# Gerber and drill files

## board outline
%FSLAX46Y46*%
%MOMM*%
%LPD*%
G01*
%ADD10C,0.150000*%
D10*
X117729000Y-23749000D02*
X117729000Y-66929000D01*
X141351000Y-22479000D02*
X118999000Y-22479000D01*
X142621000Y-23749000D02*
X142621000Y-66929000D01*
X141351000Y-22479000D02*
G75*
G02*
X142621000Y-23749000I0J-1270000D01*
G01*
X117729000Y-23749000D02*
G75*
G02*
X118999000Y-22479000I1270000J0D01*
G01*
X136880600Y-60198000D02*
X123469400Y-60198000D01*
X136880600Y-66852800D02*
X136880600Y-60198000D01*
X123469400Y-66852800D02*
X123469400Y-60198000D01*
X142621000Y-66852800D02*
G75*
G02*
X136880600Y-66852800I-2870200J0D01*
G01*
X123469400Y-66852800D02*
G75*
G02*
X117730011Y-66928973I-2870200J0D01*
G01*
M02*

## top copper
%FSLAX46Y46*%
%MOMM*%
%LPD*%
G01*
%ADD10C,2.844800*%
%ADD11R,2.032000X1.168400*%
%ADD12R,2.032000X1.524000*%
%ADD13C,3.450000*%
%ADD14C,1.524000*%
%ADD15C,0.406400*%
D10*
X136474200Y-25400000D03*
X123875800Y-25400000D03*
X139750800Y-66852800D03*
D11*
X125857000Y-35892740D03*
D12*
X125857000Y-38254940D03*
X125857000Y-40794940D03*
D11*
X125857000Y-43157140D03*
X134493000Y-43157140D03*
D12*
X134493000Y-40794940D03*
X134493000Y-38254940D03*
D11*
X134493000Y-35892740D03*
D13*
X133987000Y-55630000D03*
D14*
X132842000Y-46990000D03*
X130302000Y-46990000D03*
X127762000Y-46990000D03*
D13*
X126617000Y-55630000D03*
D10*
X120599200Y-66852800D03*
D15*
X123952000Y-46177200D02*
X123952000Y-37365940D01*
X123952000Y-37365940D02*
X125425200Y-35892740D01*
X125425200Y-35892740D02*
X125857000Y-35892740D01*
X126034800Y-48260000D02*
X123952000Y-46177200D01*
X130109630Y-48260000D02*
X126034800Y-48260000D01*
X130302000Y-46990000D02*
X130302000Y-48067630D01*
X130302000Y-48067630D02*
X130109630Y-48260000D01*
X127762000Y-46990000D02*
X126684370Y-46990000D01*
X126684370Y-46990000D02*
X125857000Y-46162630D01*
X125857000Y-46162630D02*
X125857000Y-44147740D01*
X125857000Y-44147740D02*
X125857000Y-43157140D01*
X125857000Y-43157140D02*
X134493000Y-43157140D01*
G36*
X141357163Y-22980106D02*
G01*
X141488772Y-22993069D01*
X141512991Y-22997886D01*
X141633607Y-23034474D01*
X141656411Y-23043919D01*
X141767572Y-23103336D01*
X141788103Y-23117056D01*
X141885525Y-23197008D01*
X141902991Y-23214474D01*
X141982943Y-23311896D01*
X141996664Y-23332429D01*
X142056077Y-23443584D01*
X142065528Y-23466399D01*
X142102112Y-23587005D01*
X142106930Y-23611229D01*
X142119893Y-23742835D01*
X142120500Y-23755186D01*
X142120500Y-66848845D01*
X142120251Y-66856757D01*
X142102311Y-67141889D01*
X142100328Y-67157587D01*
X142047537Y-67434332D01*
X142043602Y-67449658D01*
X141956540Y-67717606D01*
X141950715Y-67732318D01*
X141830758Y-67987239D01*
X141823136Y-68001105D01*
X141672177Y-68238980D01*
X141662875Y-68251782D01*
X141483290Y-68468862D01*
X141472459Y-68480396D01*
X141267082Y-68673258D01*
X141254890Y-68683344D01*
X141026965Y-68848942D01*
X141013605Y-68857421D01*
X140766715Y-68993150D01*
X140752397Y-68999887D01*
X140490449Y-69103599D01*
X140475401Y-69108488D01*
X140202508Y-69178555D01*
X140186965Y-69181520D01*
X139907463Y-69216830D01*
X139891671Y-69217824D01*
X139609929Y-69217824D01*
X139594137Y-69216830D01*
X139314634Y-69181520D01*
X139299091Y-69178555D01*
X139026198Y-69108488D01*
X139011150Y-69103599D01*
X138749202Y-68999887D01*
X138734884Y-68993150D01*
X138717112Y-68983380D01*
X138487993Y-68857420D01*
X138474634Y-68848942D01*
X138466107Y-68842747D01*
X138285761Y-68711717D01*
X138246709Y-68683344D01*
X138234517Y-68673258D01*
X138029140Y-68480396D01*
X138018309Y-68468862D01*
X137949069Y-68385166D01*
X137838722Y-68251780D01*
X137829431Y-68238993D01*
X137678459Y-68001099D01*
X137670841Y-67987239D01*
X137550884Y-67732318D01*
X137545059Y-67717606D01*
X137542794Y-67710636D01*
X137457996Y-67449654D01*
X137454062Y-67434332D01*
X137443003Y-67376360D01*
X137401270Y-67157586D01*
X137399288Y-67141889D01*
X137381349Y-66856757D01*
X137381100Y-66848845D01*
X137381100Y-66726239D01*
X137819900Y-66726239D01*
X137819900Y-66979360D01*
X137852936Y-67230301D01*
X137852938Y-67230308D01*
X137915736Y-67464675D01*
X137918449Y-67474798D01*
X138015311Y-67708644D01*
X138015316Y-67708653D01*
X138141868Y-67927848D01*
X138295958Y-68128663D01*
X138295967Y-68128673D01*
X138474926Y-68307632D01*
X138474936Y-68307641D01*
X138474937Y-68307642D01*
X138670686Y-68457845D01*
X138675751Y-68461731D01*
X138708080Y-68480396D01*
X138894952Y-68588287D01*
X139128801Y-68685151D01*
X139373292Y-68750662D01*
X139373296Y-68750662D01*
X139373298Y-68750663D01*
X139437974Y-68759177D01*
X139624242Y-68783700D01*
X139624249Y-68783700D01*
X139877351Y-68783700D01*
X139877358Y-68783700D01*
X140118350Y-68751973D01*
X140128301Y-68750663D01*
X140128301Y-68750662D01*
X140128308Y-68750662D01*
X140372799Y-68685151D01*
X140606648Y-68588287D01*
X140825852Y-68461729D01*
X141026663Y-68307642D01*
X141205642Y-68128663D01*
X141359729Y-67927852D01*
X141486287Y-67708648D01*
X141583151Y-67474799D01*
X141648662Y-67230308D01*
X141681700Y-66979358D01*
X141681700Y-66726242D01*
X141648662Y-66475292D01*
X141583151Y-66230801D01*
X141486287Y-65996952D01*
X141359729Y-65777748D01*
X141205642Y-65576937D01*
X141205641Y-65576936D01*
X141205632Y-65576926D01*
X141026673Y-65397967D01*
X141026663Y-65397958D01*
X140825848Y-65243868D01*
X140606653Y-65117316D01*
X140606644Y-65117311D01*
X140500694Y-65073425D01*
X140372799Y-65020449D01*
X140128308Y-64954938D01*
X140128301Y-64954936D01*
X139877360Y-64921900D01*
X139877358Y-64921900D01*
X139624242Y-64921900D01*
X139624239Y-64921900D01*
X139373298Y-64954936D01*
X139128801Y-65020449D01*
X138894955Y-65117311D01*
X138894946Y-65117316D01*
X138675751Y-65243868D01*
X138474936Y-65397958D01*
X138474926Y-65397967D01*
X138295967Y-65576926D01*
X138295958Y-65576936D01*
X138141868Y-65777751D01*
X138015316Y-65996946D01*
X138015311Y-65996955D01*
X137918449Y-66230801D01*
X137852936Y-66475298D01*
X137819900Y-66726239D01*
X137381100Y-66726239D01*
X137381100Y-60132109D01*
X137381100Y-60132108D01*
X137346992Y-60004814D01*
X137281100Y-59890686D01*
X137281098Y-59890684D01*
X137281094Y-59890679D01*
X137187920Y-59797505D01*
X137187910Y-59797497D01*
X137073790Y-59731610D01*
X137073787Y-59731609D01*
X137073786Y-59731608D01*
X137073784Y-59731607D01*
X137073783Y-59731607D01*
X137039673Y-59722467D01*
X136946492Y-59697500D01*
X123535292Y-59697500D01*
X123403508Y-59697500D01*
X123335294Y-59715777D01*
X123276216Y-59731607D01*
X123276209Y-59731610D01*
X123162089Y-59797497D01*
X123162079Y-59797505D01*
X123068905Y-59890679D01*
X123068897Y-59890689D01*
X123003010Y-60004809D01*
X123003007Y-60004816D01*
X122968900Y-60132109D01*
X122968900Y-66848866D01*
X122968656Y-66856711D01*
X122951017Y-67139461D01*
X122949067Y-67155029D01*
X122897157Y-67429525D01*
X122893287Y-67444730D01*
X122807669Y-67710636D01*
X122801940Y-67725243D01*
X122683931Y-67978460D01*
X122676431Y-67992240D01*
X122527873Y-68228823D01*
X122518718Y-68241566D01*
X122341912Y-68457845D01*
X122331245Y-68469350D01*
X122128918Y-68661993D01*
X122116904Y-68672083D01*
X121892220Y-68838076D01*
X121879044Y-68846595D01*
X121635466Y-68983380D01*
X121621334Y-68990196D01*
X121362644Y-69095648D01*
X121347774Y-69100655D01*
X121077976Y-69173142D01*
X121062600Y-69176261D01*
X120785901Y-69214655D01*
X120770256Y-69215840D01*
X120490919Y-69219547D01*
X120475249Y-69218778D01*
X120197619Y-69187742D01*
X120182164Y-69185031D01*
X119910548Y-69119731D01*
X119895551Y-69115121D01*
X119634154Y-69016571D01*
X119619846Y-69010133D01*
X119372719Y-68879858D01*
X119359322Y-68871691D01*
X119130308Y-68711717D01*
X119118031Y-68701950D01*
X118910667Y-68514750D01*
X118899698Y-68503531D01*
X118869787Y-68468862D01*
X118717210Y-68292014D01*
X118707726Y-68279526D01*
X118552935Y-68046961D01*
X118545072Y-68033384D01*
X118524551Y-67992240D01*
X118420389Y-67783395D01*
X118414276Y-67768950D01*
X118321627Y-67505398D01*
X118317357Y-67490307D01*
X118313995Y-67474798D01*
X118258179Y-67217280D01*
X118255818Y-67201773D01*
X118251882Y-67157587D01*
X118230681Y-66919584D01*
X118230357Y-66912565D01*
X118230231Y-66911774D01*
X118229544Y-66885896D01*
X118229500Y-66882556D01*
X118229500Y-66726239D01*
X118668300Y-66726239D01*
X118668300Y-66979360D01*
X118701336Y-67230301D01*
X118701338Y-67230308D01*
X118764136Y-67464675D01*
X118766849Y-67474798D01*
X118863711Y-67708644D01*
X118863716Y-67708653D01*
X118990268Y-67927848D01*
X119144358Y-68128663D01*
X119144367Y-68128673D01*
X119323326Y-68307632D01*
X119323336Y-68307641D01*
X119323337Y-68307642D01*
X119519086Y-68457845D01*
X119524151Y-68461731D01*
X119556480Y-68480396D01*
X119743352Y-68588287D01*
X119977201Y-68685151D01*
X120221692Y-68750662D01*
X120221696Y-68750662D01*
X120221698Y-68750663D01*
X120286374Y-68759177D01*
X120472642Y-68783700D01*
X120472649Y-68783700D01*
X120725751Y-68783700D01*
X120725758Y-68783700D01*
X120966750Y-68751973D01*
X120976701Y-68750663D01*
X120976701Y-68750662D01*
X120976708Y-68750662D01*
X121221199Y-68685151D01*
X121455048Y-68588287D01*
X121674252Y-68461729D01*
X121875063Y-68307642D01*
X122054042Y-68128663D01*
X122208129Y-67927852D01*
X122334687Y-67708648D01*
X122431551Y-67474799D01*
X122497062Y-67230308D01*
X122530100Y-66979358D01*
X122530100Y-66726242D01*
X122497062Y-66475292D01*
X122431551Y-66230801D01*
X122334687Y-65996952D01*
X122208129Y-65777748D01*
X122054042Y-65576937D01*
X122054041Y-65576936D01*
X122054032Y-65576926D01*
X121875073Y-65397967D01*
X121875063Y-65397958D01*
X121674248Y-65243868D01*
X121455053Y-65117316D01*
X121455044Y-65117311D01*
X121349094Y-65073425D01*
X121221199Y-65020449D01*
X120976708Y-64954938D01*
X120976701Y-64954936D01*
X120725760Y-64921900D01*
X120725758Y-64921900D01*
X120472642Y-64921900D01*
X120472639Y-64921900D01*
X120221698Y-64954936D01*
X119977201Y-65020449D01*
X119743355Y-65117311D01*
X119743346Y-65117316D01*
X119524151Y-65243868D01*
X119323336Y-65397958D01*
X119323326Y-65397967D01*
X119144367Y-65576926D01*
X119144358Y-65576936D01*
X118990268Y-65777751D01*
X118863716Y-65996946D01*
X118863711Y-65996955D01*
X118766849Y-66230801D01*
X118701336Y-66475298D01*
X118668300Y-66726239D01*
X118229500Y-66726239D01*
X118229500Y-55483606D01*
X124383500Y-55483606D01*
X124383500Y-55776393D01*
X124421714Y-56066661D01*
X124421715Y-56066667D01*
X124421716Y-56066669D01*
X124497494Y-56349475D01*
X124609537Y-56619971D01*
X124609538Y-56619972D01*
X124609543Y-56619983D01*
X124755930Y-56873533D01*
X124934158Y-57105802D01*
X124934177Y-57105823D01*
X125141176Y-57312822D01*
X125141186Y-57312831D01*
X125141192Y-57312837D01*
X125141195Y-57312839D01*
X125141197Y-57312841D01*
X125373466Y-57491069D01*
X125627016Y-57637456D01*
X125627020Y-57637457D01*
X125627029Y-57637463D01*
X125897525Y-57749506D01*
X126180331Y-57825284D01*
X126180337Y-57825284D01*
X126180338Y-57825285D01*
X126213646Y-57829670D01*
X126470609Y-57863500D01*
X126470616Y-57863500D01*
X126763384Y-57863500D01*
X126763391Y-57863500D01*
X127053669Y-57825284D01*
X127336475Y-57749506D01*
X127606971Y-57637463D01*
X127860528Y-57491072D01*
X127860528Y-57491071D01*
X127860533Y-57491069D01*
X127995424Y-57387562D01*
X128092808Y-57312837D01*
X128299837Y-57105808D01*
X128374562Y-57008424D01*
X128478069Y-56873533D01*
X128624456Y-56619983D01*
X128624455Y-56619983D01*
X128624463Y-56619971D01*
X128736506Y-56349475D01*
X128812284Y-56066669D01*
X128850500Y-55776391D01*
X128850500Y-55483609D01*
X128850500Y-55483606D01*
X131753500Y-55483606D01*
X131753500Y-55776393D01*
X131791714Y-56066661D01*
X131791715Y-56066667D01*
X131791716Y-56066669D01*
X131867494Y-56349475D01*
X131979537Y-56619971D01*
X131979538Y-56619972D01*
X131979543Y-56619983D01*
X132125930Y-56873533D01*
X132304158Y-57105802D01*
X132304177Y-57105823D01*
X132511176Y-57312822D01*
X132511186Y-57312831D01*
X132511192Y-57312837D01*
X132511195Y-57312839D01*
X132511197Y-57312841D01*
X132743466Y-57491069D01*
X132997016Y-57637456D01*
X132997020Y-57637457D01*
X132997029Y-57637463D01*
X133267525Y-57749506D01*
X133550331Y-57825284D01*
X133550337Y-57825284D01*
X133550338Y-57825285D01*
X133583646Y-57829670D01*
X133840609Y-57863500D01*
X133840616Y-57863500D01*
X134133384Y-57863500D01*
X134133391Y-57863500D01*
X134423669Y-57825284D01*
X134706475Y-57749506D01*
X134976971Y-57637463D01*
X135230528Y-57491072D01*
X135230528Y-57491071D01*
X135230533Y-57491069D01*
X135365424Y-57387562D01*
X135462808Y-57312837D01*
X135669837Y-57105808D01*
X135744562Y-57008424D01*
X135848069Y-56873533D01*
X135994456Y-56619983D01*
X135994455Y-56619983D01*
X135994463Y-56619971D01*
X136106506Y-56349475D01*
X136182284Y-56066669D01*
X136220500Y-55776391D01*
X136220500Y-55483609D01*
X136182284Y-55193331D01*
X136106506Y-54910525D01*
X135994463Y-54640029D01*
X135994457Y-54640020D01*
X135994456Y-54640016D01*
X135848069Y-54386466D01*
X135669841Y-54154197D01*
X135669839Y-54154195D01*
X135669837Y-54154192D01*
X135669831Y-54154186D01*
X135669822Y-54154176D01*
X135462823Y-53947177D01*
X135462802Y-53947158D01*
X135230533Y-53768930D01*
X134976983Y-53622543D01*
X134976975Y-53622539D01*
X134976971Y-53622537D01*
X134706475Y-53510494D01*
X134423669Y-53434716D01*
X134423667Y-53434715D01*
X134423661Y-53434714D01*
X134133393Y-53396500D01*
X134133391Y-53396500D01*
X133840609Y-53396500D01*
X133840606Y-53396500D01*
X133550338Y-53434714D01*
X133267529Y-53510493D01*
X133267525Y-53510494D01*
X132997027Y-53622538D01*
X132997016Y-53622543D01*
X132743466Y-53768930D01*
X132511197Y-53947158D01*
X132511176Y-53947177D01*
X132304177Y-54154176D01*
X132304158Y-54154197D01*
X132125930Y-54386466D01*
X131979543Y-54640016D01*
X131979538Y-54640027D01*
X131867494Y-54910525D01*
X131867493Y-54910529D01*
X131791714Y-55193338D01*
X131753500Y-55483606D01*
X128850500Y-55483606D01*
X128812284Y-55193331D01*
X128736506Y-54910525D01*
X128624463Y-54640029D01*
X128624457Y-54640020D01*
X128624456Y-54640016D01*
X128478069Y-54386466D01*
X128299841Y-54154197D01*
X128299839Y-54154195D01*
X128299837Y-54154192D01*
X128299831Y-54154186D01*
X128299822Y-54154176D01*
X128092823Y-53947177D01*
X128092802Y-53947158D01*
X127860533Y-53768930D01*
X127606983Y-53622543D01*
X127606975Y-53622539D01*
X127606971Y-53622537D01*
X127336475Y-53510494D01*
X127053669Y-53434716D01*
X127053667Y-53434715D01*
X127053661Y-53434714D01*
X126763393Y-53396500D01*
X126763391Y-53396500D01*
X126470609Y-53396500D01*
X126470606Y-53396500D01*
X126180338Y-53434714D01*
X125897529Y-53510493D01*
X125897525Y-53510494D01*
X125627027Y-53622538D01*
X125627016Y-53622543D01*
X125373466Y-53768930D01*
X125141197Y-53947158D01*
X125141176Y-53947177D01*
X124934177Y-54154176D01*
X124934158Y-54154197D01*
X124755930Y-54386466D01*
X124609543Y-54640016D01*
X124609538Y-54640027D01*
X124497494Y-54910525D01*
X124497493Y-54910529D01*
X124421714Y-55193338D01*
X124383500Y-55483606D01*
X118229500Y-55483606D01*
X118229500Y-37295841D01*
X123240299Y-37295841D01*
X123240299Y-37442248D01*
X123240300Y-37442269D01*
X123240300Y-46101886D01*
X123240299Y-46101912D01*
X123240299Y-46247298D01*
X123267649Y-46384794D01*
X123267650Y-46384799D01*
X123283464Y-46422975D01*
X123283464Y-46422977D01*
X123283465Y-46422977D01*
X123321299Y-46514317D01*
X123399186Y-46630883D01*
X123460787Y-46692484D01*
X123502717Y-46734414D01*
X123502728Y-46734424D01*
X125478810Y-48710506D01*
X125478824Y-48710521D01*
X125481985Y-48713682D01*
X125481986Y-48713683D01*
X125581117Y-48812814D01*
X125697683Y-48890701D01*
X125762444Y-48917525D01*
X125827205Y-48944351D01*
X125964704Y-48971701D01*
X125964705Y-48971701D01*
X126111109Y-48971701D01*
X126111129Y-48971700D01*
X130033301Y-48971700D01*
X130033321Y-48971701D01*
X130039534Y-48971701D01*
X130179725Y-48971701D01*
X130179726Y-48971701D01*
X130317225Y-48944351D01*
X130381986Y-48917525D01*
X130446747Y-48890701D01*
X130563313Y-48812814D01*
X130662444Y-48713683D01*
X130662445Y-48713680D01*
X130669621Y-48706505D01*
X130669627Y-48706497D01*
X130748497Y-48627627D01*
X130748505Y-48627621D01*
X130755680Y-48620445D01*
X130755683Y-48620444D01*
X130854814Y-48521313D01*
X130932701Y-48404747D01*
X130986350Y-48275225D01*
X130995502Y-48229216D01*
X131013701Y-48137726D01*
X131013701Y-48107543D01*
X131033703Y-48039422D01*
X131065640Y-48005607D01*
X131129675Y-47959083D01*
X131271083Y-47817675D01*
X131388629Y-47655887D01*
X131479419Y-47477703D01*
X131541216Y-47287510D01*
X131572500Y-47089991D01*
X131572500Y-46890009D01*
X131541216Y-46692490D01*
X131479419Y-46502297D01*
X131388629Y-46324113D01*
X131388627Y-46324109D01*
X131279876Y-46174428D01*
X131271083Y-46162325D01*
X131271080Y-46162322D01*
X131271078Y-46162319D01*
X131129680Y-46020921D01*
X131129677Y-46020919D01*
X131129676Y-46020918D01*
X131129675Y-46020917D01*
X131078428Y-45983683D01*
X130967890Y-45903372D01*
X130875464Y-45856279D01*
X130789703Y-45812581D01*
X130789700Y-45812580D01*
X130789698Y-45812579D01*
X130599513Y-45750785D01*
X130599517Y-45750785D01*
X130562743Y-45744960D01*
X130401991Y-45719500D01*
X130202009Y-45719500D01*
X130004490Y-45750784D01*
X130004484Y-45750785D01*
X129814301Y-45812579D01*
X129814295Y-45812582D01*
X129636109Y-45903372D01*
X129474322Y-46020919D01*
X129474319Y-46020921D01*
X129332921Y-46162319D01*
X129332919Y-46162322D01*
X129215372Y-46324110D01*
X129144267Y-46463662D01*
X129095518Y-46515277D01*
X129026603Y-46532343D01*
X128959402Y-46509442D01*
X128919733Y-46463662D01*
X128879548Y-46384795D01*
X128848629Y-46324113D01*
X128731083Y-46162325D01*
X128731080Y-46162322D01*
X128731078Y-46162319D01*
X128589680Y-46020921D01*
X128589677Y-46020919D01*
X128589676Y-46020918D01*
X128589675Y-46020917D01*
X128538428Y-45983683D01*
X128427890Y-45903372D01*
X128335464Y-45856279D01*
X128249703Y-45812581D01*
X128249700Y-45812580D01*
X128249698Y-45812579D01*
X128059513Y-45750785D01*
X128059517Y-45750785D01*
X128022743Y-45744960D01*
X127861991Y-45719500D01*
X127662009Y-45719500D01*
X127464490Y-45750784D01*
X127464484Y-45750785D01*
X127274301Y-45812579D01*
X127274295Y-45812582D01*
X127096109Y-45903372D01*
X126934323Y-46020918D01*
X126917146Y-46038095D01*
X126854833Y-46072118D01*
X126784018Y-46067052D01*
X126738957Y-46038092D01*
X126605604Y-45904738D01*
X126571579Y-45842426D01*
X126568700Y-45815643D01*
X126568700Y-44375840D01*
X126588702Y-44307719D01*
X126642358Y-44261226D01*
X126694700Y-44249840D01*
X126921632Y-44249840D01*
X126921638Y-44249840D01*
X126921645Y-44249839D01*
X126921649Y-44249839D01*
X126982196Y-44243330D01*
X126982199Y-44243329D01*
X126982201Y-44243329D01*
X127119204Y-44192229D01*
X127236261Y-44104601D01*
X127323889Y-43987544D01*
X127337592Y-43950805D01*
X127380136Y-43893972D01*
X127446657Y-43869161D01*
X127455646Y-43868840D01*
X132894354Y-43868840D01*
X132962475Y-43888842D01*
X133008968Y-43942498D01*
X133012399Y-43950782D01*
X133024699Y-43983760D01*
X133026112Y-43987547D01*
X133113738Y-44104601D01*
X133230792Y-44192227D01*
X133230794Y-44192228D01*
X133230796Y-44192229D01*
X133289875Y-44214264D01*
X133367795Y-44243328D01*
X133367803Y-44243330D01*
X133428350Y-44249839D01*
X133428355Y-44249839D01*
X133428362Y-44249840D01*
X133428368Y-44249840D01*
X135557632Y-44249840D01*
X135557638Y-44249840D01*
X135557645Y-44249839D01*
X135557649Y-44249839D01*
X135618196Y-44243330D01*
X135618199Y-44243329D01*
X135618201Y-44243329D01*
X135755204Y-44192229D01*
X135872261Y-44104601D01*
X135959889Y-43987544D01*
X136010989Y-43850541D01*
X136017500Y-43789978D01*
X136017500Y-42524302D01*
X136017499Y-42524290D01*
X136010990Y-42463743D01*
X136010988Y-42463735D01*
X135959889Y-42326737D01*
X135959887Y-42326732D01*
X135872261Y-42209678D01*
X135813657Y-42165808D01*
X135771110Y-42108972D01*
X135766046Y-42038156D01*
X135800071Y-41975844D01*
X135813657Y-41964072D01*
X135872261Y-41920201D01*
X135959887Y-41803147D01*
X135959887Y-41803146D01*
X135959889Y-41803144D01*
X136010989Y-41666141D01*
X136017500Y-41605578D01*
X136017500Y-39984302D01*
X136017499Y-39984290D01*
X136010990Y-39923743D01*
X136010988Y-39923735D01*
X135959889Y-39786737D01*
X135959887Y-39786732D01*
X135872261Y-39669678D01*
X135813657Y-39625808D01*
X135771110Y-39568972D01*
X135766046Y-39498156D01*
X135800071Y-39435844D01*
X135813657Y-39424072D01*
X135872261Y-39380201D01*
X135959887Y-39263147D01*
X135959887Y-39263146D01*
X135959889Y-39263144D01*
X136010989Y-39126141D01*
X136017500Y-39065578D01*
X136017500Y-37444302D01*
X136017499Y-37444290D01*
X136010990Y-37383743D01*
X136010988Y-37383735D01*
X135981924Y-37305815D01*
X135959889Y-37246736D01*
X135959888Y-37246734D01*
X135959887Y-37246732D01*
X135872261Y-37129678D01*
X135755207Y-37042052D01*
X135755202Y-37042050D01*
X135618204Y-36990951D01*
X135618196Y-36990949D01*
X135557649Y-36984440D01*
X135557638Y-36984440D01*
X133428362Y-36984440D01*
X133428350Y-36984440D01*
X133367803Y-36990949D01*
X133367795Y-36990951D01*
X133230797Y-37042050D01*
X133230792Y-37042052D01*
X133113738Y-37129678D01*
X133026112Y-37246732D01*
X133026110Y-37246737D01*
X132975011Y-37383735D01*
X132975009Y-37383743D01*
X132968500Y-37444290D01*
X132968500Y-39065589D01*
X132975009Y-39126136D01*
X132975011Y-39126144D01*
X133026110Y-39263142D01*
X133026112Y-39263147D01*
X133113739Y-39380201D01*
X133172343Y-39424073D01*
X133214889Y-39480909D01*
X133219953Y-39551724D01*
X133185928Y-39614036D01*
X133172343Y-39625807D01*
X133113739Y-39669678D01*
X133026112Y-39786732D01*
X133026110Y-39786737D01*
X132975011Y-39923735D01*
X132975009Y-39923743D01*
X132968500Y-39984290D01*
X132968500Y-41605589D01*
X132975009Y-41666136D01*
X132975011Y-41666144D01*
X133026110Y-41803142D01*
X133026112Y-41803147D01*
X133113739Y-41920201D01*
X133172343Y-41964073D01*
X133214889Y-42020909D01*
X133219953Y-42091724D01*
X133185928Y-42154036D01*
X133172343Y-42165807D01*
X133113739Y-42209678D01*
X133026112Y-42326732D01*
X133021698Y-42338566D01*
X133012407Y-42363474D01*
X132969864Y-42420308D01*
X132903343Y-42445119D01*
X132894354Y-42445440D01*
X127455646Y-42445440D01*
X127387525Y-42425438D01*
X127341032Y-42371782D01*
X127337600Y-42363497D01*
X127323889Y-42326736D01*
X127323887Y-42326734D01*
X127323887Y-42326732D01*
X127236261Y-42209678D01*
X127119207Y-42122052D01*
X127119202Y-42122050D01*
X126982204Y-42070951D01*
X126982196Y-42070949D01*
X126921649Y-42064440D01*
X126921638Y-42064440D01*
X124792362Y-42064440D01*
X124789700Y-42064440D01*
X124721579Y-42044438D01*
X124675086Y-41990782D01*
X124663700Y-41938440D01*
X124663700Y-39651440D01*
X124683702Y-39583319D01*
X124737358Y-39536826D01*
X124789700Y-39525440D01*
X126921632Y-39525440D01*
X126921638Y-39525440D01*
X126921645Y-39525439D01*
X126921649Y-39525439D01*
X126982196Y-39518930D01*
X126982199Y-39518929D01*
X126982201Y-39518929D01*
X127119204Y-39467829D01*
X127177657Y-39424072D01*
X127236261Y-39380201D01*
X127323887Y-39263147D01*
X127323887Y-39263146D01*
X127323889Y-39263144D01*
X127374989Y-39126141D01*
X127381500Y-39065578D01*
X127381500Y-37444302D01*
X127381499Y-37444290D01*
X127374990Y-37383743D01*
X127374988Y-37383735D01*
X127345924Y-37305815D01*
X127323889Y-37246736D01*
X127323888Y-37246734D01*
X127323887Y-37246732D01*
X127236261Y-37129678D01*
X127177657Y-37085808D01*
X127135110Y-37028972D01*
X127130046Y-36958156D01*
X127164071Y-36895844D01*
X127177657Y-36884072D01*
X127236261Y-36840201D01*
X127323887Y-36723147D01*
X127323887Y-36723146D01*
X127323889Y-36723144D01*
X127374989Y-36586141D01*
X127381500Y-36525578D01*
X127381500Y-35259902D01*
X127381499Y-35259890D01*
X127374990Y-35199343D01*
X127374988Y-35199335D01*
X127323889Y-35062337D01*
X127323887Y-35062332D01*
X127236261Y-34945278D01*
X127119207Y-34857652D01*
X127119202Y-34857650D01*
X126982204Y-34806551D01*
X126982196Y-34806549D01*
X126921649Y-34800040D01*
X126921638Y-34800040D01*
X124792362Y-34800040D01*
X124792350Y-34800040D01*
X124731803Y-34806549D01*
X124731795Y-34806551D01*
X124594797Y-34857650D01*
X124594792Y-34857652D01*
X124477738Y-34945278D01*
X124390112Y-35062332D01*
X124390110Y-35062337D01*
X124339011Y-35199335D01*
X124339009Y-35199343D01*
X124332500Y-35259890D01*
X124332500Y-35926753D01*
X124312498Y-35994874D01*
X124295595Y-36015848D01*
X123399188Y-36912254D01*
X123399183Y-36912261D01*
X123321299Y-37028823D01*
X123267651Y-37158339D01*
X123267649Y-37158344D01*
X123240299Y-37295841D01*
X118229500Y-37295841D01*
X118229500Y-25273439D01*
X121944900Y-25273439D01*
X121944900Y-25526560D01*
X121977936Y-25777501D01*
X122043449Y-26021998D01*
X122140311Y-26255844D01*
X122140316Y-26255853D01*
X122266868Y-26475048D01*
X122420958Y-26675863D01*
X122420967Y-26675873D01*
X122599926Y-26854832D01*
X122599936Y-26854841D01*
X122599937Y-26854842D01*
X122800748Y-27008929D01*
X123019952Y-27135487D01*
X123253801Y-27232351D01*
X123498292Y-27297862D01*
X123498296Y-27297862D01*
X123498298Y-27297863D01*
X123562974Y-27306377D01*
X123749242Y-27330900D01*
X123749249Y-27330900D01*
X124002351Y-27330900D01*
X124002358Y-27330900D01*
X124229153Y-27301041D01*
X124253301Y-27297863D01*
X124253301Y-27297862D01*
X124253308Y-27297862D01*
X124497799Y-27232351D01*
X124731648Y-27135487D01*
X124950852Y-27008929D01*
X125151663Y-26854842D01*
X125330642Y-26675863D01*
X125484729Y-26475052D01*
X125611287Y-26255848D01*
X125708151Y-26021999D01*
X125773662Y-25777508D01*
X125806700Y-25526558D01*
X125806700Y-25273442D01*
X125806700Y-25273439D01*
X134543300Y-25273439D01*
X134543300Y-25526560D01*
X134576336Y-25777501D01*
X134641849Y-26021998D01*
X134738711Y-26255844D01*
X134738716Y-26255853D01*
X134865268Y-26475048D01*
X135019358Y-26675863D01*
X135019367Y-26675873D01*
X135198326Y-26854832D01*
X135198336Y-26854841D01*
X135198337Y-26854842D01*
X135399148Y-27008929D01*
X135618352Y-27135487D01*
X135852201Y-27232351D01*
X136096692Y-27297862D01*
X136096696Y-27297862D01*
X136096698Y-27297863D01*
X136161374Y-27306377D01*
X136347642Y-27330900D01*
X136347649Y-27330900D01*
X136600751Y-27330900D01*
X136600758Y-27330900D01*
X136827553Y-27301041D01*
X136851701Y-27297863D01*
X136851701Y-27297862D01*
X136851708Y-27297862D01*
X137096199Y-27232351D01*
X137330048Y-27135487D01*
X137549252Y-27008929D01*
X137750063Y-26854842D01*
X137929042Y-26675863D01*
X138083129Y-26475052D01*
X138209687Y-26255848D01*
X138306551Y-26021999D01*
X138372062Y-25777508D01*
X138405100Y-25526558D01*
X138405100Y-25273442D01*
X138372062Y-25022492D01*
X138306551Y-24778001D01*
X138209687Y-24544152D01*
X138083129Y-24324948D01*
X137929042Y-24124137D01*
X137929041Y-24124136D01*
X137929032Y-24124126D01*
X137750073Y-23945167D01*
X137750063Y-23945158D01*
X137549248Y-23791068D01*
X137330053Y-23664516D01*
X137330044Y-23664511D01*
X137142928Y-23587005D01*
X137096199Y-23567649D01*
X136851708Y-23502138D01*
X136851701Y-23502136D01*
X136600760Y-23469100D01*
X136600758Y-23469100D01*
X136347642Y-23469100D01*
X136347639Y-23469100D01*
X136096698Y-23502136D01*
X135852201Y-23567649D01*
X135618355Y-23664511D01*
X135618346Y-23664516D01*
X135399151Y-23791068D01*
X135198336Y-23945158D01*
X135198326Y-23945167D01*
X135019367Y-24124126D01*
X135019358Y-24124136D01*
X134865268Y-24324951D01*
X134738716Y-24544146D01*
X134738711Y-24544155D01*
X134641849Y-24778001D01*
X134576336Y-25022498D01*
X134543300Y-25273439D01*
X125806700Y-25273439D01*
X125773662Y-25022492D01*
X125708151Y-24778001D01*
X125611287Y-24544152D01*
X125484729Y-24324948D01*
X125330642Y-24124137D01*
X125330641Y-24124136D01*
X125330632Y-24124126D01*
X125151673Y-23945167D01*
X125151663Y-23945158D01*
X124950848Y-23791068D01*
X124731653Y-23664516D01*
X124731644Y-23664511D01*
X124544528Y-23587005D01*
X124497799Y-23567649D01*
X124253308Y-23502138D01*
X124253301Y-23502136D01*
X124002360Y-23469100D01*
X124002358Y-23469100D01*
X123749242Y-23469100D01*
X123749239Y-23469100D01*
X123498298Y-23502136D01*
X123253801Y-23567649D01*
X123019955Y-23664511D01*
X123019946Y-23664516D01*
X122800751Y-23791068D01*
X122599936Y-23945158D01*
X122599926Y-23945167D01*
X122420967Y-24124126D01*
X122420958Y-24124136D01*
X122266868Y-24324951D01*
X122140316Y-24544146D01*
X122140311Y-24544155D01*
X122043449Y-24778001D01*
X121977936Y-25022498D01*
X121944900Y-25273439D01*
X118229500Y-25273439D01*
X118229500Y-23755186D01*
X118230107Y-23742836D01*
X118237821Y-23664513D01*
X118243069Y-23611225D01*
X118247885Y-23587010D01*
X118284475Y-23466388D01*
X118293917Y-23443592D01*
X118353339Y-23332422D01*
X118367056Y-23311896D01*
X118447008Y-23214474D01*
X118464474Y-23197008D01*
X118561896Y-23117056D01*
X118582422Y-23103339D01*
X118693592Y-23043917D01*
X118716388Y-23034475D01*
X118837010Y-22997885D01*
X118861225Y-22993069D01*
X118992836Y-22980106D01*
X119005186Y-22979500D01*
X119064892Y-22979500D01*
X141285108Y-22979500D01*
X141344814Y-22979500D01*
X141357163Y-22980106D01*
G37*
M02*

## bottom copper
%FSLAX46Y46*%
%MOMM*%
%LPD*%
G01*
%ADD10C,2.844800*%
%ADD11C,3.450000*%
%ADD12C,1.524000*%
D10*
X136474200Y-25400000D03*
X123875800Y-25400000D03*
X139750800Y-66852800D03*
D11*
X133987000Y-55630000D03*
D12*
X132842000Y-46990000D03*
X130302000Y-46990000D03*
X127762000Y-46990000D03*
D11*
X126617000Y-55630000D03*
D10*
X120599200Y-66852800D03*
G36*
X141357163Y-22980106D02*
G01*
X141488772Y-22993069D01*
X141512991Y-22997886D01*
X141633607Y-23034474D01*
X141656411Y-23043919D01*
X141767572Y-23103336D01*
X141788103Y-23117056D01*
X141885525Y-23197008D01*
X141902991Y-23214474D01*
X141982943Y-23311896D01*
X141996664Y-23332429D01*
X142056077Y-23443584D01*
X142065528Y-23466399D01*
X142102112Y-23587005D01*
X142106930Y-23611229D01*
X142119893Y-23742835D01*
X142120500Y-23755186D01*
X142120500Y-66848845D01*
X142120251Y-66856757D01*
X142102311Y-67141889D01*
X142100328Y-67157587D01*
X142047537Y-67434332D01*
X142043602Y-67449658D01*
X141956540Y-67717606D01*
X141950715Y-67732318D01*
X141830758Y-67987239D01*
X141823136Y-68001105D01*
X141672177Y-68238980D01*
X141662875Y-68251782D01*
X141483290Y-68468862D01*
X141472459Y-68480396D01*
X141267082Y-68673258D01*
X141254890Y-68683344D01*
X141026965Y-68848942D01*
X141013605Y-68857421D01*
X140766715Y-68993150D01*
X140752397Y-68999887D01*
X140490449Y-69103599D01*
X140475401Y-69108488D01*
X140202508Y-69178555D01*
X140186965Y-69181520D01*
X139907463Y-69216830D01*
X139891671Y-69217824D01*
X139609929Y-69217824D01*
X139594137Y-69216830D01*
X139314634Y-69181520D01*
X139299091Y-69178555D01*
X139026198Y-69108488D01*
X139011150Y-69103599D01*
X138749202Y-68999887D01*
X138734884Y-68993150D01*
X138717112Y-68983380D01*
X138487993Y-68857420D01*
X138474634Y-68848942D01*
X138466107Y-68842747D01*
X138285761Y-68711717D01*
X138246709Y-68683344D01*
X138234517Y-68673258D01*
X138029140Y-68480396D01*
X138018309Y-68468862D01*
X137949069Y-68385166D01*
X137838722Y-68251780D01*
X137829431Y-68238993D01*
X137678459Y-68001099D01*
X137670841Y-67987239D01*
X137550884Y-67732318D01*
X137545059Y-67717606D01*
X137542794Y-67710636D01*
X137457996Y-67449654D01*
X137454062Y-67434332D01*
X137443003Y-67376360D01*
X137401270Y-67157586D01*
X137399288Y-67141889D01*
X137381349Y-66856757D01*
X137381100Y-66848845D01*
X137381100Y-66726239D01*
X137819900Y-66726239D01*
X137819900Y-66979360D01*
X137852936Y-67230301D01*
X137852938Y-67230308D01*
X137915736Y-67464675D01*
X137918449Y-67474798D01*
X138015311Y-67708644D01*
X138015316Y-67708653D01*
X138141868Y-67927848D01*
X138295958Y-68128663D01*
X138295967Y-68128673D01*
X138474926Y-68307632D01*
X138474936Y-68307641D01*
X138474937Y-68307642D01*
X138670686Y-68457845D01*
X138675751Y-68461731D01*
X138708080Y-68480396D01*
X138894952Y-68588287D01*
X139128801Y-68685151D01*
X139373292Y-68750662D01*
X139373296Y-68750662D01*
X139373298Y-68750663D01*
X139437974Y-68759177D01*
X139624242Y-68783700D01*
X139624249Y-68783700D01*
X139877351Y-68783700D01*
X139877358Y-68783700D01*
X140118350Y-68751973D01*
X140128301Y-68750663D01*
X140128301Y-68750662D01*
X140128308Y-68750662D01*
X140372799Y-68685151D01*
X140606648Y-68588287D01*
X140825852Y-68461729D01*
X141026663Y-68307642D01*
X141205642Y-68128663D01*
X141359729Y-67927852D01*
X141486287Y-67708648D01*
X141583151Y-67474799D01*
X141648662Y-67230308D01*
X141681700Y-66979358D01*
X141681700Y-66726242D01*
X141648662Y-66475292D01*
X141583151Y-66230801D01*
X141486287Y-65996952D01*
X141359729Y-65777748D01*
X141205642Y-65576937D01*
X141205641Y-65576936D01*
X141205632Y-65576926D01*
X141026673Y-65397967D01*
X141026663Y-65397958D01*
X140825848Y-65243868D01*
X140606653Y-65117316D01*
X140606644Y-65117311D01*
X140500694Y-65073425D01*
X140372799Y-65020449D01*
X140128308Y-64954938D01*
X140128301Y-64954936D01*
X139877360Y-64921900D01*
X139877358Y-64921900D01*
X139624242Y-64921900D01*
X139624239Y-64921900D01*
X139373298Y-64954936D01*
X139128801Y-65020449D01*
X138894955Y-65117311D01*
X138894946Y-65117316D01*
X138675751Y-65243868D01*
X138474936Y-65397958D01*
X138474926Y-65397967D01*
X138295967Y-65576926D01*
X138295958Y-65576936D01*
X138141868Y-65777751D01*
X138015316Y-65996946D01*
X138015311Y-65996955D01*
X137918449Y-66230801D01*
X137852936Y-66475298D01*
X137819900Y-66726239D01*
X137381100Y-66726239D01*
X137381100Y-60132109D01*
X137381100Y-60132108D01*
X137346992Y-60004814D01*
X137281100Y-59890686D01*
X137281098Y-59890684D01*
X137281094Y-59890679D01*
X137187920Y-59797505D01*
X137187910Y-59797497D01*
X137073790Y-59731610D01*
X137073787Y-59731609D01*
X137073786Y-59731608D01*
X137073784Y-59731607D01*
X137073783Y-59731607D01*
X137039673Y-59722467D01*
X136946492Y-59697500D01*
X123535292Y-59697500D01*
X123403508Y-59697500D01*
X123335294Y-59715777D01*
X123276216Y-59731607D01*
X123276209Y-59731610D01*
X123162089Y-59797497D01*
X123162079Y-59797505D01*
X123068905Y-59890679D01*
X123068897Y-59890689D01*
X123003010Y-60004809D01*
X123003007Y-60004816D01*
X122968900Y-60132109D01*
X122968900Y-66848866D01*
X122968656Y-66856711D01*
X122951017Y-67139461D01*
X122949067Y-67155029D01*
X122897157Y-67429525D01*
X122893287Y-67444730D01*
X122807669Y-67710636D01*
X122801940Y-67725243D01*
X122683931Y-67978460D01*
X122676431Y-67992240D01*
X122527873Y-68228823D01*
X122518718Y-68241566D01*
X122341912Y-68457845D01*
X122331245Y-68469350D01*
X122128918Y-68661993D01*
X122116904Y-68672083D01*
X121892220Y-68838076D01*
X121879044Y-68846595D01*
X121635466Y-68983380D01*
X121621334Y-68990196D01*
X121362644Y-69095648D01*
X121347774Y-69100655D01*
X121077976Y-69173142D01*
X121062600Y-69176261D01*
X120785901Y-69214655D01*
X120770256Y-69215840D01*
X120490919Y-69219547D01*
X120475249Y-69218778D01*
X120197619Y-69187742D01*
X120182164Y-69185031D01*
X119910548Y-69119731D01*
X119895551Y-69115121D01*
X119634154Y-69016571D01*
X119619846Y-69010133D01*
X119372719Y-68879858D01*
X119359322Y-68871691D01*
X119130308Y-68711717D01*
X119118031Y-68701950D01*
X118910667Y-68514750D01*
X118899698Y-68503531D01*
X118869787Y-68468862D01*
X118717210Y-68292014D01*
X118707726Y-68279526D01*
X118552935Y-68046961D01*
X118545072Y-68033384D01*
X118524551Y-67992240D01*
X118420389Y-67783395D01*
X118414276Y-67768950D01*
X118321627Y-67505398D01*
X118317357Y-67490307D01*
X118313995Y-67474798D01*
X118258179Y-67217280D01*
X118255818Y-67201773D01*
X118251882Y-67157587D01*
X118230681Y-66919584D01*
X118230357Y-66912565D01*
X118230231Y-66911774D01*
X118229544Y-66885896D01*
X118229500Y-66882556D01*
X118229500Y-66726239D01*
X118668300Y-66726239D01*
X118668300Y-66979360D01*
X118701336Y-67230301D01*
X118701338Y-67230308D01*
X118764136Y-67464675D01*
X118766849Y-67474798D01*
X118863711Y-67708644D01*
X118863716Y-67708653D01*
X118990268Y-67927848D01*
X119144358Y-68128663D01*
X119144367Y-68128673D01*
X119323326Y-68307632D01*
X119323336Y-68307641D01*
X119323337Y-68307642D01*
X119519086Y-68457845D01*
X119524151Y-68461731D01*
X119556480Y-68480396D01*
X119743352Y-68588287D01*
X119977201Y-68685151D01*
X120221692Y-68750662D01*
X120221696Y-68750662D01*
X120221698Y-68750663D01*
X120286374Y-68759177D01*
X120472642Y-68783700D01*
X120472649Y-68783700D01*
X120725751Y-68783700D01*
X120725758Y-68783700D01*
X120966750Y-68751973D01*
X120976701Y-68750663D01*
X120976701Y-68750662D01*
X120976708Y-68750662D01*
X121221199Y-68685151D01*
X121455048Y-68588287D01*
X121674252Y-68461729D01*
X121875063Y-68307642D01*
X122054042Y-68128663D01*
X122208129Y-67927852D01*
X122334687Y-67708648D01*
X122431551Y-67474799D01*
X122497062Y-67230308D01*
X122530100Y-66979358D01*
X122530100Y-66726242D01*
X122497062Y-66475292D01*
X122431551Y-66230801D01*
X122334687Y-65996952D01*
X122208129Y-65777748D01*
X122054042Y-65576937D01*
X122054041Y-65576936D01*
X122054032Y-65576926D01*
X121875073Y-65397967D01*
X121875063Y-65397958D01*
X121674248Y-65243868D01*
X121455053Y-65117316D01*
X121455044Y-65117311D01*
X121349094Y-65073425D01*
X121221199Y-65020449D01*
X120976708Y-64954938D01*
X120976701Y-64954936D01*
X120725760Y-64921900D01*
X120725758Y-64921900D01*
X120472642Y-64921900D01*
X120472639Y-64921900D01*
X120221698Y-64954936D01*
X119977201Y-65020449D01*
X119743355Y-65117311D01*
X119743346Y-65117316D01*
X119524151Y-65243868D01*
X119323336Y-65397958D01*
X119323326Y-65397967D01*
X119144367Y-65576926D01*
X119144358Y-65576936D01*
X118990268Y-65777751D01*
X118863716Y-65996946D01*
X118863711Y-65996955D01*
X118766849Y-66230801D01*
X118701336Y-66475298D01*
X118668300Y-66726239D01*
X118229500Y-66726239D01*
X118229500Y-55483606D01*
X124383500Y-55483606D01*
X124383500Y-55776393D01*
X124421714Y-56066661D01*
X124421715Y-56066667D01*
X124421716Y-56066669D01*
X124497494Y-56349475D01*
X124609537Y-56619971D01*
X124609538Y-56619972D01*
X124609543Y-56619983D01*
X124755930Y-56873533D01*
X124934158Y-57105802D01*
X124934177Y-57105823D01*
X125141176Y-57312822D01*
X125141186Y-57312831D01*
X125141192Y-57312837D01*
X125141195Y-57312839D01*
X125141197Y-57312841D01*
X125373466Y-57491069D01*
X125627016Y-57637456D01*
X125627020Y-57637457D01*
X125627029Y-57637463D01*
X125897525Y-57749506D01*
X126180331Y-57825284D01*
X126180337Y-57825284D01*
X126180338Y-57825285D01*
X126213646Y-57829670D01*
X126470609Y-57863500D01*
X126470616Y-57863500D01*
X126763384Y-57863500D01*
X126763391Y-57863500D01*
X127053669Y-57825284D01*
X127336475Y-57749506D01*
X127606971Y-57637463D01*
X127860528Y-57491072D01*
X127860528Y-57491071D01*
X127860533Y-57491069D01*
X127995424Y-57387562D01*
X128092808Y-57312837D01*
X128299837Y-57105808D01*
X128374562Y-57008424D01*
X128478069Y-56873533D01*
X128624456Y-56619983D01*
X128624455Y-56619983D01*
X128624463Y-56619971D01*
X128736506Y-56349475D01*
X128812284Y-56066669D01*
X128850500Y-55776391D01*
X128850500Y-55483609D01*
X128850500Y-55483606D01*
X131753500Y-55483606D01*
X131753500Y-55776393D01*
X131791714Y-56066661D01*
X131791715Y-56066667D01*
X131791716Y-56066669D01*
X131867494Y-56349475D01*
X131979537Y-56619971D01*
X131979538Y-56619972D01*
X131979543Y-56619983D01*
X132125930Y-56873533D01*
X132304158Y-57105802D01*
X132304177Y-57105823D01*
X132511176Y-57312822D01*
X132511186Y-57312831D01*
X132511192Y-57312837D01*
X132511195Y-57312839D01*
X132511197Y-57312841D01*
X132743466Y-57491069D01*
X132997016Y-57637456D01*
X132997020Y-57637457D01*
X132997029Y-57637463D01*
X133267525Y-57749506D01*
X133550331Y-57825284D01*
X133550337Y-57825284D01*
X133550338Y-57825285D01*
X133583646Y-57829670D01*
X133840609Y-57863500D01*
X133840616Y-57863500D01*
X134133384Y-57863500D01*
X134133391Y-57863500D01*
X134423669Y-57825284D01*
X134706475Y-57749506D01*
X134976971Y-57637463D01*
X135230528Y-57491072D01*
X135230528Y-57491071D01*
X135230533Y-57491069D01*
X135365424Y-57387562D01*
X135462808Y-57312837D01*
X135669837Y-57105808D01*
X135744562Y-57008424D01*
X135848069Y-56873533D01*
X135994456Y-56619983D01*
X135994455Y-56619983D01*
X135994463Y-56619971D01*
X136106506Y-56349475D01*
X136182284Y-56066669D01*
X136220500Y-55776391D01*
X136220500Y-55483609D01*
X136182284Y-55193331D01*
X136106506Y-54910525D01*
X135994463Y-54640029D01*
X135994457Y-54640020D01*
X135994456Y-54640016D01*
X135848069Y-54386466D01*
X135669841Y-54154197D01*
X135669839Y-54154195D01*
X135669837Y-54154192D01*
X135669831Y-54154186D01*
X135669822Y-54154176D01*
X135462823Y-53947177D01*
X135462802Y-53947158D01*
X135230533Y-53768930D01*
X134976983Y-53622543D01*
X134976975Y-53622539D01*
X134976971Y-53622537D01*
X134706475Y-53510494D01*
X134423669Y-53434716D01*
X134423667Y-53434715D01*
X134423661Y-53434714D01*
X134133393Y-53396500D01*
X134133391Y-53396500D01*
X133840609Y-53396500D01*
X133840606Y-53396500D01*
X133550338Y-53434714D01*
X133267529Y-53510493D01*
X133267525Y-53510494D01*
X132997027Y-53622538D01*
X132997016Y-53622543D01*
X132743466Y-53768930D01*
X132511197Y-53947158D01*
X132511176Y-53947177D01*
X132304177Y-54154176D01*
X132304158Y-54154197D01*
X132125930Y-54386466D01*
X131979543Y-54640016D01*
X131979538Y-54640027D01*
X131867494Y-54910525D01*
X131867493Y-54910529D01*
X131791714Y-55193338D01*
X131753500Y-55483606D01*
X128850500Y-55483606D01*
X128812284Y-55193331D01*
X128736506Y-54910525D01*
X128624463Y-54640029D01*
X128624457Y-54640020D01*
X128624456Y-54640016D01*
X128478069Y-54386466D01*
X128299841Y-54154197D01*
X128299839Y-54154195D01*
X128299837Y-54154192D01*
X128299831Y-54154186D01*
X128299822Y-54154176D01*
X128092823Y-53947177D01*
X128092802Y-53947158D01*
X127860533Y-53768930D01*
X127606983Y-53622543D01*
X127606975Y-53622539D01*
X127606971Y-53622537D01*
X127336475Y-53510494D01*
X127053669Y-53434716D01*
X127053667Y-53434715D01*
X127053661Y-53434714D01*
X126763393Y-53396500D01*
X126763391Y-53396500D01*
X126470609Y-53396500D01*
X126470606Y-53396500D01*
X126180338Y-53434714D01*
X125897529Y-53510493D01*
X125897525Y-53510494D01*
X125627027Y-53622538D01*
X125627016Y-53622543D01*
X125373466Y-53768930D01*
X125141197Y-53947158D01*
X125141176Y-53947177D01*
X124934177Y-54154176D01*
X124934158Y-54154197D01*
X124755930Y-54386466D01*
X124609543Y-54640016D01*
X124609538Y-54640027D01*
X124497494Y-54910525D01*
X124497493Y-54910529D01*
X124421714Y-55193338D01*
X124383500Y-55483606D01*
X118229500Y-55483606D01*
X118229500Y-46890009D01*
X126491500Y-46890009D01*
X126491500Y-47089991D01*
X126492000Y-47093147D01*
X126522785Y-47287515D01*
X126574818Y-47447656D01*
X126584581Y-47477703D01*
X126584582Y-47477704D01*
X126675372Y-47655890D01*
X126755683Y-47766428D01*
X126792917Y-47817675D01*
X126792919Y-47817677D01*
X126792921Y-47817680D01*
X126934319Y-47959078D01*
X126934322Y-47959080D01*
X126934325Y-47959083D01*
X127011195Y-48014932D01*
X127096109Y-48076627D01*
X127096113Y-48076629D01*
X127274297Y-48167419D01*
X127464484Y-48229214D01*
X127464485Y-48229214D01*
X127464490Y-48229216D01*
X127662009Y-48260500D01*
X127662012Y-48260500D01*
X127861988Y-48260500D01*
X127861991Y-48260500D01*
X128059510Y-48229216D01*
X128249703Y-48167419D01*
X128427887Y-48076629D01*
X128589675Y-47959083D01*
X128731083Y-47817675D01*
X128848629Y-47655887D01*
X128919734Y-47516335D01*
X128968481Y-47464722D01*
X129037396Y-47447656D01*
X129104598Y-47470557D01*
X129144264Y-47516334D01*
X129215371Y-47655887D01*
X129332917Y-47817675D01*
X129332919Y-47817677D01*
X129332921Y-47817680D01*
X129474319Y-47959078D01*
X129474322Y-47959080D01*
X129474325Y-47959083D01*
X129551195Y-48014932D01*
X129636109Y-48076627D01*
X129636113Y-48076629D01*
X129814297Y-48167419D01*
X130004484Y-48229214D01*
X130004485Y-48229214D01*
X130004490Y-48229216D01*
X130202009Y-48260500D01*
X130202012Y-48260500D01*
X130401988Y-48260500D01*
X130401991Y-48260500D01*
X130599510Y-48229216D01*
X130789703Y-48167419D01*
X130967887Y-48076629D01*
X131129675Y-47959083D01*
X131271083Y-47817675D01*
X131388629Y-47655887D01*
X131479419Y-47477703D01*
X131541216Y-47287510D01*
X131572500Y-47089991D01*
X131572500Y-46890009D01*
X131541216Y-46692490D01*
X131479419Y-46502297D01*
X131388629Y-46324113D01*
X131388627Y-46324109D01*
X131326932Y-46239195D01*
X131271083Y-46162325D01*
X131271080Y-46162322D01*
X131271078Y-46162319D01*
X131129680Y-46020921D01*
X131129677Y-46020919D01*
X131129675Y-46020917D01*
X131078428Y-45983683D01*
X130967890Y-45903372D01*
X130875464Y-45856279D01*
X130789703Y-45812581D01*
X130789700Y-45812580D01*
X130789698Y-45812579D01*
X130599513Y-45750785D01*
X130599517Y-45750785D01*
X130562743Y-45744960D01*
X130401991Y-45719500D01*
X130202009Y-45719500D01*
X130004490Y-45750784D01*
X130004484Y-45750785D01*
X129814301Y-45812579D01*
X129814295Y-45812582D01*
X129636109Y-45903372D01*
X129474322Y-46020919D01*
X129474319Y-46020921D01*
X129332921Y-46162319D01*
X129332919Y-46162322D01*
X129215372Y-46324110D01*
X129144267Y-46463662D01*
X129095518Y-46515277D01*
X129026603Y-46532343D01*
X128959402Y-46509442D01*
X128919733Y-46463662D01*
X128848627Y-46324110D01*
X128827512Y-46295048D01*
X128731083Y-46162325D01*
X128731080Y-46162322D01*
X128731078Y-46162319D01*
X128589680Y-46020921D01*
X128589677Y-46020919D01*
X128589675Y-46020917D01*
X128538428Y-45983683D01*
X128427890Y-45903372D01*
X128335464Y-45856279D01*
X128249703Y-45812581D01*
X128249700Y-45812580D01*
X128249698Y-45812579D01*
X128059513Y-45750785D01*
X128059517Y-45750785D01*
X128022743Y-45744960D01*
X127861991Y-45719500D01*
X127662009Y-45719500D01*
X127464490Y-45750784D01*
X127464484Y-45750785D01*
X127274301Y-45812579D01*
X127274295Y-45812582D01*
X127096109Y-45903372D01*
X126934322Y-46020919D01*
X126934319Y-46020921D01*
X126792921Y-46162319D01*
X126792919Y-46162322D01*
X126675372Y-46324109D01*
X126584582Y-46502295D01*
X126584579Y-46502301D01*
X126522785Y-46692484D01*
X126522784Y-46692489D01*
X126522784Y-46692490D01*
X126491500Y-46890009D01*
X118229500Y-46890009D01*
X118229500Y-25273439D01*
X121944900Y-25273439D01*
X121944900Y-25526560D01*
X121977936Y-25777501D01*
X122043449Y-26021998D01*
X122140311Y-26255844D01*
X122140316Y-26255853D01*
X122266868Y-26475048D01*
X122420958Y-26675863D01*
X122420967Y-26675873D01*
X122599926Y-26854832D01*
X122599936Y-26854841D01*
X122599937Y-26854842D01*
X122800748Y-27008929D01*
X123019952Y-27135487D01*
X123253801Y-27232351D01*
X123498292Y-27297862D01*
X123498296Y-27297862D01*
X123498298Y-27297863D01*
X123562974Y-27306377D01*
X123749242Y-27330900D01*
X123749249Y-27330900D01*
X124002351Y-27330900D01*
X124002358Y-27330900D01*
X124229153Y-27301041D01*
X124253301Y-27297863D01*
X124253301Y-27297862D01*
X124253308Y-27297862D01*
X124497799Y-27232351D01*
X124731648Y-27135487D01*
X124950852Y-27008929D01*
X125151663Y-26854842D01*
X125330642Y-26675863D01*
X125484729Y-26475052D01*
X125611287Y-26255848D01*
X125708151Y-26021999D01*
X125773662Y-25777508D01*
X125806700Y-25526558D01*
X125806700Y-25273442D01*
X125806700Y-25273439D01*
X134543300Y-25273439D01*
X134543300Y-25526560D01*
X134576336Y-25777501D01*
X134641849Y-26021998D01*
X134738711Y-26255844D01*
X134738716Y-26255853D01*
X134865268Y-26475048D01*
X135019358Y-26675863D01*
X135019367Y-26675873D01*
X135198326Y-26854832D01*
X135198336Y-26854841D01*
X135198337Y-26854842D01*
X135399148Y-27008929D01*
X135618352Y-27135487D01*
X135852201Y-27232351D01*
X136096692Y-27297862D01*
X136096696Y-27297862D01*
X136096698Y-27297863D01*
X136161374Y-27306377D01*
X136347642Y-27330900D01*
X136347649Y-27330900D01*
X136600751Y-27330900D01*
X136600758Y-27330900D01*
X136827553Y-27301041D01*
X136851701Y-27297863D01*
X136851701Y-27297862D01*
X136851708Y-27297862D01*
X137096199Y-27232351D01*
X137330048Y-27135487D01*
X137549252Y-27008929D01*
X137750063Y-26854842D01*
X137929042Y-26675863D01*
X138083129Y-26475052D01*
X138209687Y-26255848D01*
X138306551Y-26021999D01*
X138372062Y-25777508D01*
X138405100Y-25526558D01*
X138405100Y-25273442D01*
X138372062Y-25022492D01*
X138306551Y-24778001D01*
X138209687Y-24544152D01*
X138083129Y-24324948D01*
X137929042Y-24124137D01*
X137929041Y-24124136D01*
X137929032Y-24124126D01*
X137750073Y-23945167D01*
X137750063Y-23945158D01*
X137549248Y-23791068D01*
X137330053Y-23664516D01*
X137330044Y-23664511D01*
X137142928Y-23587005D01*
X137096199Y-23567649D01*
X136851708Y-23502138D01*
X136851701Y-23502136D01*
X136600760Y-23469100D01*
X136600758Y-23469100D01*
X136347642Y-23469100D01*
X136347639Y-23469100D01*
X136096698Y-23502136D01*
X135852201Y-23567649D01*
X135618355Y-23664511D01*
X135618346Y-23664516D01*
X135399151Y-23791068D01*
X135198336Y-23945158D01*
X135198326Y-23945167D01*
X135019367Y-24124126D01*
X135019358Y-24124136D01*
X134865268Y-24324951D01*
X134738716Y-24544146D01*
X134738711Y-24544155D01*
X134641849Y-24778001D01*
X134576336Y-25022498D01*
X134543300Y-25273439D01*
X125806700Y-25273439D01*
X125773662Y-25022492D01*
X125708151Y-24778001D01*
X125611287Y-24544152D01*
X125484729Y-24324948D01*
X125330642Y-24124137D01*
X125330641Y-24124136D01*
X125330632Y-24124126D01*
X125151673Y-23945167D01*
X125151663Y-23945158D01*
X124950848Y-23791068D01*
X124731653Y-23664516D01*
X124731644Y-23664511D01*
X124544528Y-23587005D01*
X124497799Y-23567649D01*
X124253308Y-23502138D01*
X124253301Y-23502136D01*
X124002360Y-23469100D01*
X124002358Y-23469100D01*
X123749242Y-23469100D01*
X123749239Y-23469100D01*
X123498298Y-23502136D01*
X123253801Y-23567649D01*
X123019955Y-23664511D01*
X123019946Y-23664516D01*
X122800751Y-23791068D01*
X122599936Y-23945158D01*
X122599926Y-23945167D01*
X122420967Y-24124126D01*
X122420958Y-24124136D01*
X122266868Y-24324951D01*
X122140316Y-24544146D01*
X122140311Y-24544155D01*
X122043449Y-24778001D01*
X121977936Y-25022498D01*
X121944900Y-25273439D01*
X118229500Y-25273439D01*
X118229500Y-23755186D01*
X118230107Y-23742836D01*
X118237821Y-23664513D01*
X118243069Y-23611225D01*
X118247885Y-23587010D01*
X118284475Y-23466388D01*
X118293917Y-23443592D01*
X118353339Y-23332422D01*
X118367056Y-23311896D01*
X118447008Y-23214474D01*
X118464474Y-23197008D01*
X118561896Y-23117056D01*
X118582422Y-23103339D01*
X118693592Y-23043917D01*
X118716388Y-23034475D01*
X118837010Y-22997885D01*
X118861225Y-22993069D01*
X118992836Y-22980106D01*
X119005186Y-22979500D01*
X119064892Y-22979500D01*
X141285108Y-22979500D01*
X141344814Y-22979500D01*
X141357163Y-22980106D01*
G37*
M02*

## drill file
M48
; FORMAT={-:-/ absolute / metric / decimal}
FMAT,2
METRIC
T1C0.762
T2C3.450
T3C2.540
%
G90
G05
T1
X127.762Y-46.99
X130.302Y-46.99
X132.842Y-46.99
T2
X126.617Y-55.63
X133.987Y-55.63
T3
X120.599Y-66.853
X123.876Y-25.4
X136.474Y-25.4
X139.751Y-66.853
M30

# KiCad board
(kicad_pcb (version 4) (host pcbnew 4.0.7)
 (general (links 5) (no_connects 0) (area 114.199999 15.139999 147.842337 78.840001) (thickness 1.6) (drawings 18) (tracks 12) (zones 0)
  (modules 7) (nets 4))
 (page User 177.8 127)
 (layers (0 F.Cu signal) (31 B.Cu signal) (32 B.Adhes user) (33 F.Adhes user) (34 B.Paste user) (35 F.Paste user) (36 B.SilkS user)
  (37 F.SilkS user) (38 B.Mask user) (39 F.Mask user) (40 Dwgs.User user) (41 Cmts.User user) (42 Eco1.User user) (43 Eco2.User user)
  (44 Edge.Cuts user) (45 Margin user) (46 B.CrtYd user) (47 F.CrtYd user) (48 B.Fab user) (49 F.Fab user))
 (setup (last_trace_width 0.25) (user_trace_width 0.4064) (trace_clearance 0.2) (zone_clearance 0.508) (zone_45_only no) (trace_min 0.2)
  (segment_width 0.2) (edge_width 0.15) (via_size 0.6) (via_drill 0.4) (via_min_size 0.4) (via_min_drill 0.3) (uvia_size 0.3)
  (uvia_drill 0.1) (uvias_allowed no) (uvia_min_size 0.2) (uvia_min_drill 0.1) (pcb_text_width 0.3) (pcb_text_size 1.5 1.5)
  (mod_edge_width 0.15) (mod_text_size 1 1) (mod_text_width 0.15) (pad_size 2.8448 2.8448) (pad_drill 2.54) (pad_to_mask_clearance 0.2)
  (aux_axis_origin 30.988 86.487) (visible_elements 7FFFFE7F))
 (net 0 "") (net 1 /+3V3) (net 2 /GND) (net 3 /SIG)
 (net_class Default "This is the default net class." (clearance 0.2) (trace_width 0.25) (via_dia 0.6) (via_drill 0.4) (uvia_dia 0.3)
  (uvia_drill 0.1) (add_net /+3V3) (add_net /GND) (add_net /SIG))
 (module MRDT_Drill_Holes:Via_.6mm (layer F.Cu) (at 146.685 42.291)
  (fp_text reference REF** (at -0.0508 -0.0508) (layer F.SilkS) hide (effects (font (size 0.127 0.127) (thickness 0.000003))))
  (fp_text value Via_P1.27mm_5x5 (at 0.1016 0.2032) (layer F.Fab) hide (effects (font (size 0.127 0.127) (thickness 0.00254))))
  (pad "" np_thru_hole circle (at -10.2108 -16.891) (size 2.8448 2.8448) (drill 2.54) (layers *.Cu *.Mask) (zone_connect 2)))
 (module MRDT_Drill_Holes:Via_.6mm (layer F.Cu) (at 142.875 43.942)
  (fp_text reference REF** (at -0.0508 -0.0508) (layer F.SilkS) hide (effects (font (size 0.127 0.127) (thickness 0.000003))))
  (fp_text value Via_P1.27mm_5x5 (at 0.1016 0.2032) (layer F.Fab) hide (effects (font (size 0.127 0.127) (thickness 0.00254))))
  (pad "" np_thru_hole circle (at -18.9992 -18.542) (size 2.8448 2.8448) (drill 2.54) (layers *.Cu *.Mask) (zone_connect 2)))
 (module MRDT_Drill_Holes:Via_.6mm (layer F.Cu) (at 146.431 49.403)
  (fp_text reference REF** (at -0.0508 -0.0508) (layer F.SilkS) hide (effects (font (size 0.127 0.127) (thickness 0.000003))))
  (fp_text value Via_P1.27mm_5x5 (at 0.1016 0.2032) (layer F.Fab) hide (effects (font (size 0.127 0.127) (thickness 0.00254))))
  (pad "" np_thru_hole circle (at -6.6802 17.4498) (size 2.8448 2.8448) (drill 2.54) (layers *.Cu *.Mask) (zone_connect 2)))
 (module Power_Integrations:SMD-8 (layer F.Cu) (at 130.175 39.52494 270)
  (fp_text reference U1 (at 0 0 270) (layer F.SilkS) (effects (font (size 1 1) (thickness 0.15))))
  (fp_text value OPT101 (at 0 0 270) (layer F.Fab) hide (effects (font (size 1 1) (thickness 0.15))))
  (pad 1 smd rect (at -3.6322 4.318 270) (size 1.1684 2.032) (layers F.Cu F.Paste F.Mask) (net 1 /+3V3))
  (pad 2 smd rect (at -1.27 4.318 270) (size 1.524 2.032) (layers F.Cu F.Paste F.Mask))
  (pad 3 smd rect (at 1.27 4.318 270) (size 1.524 2.032) (layers F.Cu F.Paste F.Mask) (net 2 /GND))
  (pad 4 smd rect (at 3.6322 4.318 270) (size 1.1684 2.032) (layers F.Cu F.Paste F.Mask) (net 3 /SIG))
  (pad 5 smd rect (at 3.6322 -4.318 270) (size 1.1684 2.032) (layers F.Cu F.Paste F.Mask) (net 3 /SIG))
  (pad 6 smd rect (at 1.27 -4.318 270) (size 1.524 2.032) (layers F.Cu F.Paste F.Mask))
  (pad 7 smd rect (at -1.27 -4.318 270) (size 1.524 2.032) (layers F.Cu F.Paste F.Mask))
  (pad 8 smd rect (at -3.6322 -4.318 270) (size 1.1684 2.032) (layers F.Cu F.Paste F.Mask) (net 2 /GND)))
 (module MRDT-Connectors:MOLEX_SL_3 (layer F.Cu) (at 130.302 46.99 180)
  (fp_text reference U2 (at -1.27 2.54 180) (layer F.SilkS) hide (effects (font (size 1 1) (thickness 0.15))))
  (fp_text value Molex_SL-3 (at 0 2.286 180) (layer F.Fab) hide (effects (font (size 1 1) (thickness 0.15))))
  (pad "" thru_hole circle (at -3.685 -8.64 180) (size 3.45 3.45) (drill 3.45) (layers *.Cu *.Mask))
  (pad 1 thru_hole circle (at -2.54 0 180) (size 1.524 1.524) (drill 0.762) (layers *.Cu *.Mask) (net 2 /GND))
  (pad 2 thru_hole circle (at 0 0 180) (size 1.524 1.524) (drill 0.762) (layers *.Cu *.Mask) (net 1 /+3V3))
  (pad 3 thru_hole circle (at 2.54 0 180) (size 1.524 1.524) (drill 0.762) (layers *.Cu *.Mask) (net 3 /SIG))
  (pad "" thru_hole circle (at 3.685 -8.64 180) (size 3.45 3.45) (drill 3.45) (layers *.Cu *.Mask)))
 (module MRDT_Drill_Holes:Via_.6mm (layer F.Cu) (at 125.984 48.514)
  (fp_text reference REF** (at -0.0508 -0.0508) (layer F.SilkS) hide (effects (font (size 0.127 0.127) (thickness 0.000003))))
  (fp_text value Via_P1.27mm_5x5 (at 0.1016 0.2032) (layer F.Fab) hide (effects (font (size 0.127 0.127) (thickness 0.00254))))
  (pad "" np_thru_hole circle (at -5.3848 18.3388) (size 2.8448 2.8448) (drill 2.54) (layers *.Cu *.Mask) (zone_connect 2)))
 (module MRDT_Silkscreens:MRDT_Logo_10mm (layer B.Cu) (at 135.509 32.766 270)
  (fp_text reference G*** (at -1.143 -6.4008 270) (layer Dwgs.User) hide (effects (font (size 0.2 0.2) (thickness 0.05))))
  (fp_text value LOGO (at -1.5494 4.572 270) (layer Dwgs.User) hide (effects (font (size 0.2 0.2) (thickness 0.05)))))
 (gr_line (start 117.729 23.749) (end 117.729 66.929) (layer Edge.Cuts) (width 0.15))
 (gr_line (start 141.351 22.479) (end 118.999 22.479) (layer Edge.Cuts) (width 0.15))
 (gr_line (start 142.621 23.749) (end 142.621 66.929) (layer Edge.Cuts) (width 0.15))
 (gr_arc (start 141.351 23.749) (end 141.351 22.479) (angle 90) (layer Edge.Cuts) (width 0.15))
 (gr_arc (start 118.999 23.749) (end 117.729 23.749) (angle 90) (layer Edge.Cuts) (width 0.15))
 (gr_line (start 136.8806 60.198) (end 123.4694 60.198) (layer Edge.Cuts) (width 0.15))
 (gr_line (start 136.8806 66.8528) (end 136.8806 60.198) (layer Edge.Cuts) (width 0.15))
 (gr_line (start 123.4694 66.8528) (end 123.4694 60.198) (layer Edge.Cuts) (width 0.15))
 (gr_arc (start 139.7508 66.8528) (end 142.621 66.8528) (angle 180) (layer Edge.Cuts) (width 0.15))
 (gr_arc (start 120.5992 66.8528) (end 123.4694 66.8528) (angle 178.4792303) (layer Edge.Cuts) (width 0.15))
 (segment (start 123.952 46.1772) (end 123.952 37.36594) (width 0.4064) (layer F.Cu) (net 1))
 (segment (start 123.952 37.36594) (end 125.4252 35.89274) (width 0.4064) (layer F.Cu) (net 1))
 (segment (start 125.4252 35.89274) (end 125.857 35.89274) (width 0.4064) (layer F.Cu) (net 1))
 (segment (start 126.0348 48.26) (end 123.952 46.1772) (width 0.4064) (layer F.Cu) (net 1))
 (segment (start 130.10963 48.26) (end 126.0348 48.26) (width 0.4064) (layer F.Cu) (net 1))
 (segment (start 130.302 46.99) (end 130.302 48.06763) (width 0.4064) (layer F.Cu) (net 1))
 (segment (start 130.302 48.06763) (end 130.10963 48.26) (width 0.4064) (layer F.Cu) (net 1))
 (segment (start 127.762 46.99) (end 126.68437 46.99) (width 0.4064) (layer F.Cu) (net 3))
 (segment (start 126.68437 46.99) (end 125.857 46.16263) (width 0.4064) (layer F.Cu) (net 3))
 (segment (start 125.857 46.16263) (end 125.857 44.14774) (width 0.4064) (layer F.Cu) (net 3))
 (segment (start 125.857 44.14774) (end 125.857 43.15714) (width 0.4064) (layer F.Cu) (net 3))
 (segment (start 125.857 43.15714) (end 134.493 43.15714) (width 0.4064) (layer F.Cu) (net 3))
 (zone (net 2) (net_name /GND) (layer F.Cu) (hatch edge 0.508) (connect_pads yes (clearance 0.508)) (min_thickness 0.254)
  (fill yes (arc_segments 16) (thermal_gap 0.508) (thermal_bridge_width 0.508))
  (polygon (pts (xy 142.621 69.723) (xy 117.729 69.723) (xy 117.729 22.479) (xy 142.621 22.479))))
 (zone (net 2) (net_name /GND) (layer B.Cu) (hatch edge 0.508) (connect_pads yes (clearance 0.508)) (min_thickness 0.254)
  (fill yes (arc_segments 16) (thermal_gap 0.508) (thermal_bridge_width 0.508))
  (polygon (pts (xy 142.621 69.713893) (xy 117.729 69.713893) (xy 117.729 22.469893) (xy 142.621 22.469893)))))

